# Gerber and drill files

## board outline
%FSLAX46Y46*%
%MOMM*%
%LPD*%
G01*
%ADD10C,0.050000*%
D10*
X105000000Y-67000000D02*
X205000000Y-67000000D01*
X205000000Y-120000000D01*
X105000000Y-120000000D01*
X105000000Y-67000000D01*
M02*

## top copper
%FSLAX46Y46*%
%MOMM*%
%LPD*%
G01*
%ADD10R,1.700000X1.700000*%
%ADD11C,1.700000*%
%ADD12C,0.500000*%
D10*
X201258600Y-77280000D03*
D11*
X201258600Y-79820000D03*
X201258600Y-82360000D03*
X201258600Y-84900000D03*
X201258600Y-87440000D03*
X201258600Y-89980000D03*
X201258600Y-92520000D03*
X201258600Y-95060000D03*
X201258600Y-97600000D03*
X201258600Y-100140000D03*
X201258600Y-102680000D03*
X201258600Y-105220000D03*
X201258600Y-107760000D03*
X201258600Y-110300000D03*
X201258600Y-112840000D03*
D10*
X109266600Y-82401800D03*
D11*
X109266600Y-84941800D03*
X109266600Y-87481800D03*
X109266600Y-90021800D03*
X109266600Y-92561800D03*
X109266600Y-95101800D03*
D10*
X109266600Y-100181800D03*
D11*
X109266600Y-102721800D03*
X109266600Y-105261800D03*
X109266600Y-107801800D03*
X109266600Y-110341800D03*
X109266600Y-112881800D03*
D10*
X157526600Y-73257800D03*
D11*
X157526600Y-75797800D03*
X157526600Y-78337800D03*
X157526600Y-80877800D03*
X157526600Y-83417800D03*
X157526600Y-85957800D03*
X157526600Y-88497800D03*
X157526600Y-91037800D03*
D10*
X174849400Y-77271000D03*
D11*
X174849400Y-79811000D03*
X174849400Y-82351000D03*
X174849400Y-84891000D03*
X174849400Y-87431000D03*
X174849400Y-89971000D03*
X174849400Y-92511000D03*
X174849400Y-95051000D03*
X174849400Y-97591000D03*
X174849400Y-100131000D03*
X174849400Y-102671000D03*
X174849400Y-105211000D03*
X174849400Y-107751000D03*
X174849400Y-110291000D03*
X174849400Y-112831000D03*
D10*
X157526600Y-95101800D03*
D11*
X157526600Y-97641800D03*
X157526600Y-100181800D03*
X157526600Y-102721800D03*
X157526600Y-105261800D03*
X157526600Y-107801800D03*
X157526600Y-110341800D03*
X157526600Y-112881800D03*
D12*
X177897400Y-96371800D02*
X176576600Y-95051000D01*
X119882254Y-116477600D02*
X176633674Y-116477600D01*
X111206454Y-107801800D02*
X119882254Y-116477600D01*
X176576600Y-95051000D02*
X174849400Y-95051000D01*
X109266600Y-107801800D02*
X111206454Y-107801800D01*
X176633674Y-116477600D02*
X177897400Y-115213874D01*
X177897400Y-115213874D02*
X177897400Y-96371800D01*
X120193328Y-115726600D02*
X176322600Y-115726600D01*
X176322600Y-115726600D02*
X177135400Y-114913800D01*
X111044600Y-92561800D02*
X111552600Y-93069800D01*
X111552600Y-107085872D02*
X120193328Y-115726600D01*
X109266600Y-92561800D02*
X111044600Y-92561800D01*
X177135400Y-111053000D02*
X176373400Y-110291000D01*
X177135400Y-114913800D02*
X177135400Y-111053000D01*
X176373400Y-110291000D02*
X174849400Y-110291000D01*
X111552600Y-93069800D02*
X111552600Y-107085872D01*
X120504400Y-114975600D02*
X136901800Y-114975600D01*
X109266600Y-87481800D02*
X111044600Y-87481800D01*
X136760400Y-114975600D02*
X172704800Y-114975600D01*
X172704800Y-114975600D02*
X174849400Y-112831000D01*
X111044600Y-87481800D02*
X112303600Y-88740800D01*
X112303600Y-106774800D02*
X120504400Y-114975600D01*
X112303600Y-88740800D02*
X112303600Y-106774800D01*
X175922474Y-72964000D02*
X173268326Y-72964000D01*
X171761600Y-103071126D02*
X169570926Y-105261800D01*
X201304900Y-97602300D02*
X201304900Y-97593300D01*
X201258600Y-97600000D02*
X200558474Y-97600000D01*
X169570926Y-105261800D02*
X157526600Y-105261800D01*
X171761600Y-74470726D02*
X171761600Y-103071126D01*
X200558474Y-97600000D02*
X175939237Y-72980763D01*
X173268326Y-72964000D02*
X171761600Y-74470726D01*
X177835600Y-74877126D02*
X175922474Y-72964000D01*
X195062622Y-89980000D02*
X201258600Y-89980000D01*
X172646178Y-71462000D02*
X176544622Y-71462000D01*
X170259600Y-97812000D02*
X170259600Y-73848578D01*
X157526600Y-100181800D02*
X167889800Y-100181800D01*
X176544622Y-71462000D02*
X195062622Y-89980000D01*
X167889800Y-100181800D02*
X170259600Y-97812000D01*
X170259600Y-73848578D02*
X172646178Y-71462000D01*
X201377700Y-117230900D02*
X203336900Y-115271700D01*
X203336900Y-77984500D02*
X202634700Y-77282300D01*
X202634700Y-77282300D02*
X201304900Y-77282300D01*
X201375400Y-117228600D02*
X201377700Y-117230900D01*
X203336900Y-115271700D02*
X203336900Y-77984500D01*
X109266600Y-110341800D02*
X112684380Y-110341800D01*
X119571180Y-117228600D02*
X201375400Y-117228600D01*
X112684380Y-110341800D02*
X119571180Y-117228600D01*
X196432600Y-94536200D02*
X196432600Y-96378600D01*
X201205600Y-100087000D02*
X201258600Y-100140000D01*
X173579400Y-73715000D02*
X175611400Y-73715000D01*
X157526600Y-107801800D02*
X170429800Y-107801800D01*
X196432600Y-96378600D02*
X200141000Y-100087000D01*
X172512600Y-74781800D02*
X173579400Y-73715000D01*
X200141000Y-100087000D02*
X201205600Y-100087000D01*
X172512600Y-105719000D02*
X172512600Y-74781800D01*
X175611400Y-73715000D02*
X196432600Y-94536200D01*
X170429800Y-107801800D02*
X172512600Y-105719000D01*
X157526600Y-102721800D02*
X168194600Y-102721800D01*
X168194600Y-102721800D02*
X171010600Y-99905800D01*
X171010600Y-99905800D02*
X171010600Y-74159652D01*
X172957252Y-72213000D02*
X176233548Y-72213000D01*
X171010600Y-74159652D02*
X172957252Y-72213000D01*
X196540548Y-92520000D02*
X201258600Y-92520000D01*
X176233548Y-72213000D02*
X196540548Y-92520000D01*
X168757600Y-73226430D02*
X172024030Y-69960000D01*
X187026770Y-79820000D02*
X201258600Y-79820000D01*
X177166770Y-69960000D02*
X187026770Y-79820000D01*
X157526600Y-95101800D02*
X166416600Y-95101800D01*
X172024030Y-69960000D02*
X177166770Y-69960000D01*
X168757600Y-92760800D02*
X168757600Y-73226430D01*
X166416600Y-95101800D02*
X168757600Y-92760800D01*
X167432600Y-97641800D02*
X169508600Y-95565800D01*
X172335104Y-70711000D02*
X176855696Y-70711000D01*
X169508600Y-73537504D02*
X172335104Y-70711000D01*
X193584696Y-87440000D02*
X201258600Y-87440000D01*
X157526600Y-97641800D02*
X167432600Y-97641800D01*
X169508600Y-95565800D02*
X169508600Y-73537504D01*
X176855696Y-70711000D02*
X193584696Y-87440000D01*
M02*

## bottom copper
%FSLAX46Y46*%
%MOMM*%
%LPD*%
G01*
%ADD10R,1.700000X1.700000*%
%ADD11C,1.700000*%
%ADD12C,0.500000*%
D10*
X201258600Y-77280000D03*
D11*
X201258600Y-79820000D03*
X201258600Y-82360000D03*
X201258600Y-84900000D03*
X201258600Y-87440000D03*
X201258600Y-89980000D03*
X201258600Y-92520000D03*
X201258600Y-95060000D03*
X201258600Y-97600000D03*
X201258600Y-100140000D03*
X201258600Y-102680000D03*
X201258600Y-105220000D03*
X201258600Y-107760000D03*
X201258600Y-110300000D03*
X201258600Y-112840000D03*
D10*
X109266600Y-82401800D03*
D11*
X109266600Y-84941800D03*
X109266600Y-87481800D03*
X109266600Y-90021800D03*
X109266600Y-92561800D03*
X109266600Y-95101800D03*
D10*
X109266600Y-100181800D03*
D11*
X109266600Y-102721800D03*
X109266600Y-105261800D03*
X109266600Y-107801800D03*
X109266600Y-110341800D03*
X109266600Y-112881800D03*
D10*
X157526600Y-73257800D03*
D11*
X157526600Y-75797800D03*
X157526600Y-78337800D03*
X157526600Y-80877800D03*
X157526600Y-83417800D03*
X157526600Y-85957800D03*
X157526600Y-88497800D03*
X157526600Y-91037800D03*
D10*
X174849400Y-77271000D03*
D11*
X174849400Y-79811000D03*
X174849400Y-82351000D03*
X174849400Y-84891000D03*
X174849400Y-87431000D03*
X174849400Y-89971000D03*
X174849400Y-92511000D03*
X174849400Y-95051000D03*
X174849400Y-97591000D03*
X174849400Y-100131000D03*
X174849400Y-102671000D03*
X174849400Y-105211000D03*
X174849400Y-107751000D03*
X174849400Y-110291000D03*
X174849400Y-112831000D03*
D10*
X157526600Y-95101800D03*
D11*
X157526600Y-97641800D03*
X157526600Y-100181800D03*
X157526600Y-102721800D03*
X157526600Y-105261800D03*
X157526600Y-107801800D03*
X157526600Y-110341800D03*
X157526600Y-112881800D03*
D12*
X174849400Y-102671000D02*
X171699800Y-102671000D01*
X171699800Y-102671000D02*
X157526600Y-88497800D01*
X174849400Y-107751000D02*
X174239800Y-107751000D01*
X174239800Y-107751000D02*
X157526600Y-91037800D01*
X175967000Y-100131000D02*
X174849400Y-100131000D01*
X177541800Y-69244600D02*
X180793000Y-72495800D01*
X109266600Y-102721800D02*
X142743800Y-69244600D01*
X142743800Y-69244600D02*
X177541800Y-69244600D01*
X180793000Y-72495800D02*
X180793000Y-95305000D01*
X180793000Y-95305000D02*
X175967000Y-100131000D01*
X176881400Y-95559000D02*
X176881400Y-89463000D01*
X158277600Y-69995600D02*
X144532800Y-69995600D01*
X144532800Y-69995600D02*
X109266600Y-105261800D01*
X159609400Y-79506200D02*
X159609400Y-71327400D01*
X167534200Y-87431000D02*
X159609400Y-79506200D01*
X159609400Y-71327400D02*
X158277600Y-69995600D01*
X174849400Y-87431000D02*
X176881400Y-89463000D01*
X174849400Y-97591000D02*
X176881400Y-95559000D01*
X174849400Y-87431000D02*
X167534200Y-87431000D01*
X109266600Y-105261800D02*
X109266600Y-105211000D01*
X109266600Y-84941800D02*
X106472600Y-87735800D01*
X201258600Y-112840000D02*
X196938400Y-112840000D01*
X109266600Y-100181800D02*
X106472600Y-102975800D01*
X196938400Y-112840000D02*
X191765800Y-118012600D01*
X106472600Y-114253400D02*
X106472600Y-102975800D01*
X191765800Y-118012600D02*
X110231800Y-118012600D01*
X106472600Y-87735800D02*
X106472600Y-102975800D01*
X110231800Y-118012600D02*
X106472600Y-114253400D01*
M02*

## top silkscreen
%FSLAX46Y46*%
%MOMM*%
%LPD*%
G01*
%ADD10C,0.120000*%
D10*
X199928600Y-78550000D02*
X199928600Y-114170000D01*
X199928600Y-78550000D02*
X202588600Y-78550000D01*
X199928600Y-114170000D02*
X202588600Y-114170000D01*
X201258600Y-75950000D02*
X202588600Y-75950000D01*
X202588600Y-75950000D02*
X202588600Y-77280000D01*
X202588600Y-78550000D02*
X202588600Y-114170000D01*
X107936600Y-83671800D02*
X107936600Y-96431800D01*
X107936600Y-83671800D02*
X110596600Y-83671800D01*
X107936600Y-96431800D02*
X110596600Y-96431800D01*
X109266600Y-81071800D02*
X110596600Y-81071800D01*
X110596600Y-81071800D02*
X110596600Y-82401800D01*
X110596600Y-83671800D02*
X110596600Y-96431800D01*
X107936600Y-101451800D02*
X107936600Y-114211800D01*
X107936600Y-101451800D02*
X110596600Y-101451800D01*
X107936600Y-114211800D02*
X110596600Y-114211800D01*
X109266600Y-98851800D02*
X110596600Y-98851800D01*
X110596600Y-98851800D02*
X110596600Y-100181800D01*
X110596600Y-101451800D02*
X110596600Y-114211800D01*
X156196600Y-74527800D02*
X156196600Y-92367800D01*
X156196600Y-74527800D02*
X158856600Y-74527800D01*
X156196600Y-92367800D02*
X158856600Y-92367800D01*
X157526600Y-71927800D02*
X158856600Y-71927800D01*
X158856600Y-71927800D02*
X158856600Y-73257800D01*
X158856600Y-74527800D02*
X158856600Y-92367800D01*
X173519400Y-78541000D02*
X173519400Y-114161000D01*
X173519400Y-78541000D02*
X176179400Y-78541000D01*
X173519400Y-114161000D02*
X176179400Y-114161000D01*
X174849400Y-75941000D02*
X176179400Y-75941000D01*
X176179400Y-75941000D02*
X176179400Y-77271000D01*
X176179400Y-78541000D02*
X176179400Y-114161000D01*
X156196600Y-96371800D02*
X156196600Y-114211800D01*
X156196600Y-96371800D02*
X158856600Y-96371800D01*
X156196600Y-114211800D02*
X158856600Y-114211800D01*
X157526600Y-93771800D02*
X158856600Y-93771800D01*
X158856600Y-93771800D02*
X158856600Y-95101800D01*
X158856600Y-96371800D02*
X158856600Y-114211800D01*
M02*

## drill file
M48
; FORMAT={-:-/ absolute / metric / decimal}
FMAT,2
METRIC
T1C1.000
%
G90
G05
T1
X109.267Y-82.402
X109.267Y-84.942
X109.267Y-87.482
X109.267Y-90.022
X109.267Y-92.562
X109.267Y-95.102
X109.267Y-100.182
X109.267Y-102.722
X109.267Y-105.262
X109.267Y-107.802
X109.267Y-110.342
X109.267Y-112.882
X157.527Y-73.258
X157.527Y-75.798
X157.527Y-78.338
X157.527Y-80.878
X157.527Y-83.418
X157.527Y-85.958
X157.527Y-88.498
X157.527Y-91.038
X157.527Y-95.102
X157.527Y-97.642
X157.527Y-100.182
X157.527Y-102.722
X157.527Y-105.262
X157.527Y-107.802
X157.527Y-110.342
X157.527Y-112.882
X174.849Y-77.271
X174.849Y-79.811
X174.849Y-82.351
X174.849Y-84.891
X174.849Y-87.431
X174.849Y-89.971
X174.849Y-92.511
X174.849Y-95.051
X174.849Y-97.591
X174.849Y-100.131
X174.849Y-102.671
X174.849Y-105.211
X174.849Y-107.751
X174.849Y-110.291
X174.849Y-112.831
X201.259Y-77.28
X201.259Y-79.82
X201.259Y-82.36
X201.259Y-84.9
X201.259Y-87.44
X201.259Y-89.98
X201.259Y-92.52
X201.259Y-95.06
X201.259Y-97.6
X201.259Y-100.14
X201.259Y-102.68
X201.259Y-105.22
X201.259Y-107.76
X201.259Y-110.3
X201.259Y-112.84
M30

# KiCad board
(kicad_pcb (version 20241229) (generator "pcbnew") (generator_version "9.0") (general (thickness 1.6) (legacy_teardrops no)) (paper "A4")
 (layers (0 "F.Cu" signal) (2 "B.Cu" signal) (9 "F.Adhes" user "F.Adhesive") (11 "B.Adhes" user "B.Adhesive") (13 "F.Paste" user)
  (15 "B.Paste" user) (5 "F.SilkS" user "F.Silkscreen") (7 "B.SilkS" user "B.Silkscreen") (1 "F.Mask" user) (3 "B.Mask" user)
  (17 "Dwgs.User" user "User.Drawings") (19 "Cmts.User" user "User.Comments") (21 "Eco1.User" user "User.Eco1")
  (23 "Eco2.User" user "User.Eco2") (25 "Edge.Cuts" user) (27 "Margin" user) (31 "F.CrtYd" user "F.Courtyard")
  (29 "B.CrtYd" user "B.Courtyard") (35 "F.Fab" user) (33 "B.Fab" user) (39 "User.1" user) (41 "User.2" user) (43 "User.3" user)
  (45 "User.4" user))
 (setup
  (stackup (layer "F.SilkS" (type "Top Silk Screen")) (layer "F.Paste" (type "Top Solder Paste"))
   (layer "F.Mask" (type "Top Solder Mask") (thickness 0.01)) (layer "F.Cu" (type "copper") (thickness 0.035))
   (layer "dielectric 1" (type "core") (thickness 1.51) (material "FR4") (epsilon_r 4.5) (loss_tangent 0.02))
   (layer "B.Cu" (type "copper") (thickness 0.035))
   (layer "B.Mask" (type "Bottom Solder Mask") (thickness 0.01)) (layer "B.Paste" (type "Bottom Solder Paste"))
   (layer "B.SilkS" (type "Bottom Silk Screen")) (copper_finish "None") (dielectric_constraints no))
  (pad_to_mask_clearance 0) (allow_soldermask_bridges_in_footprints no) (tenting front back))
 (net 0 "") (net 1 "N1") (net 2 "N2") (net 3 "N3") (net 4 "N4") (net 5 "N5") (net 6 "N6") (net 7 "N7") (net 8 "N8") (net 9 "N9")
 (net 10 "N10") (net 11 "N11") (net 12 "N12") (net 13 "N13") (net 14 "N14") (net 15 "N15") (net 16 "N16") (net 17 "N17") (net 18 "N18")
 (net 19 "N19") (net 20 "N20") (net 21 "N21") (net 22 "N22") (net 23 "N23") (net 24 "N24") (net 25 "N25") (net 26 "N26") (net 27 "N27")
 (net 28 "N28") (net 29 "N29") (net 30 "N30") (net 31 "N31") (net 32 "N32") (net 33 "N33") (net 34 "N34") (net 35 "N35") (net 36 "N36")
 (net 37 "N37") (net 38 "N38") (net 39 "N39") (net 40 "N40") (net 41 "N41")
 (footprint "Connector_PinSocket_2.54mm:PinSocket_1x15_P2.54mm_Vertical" (layer "F.Cu") (at 201.2586 77.28)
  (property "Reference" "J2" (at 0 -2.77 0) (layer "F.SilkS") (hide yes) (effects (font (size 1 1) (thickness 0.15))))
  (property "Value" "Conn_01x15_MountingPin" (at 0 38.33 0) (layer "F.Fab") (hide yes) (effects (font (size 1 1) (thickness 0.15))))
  (fp_line (start -1.33 1.27) (end -1.33 36.89) (stroke (width 0.12) (type solid)) (layer "F.SilkS"))
  (fp_line (start -1.33 1.27) (end 1.33 1.27) (stroke (width 0.12) (type solid)) (layer "F.SilkS"))
  (fp_line (start -1.33 36.89) (end 1.33 36.89) (stroke (width 0.12) (type solid)) (layer "F.SilkS"))
  (fp_line (start 0 -1.33) (end 1.33 -1.33) (stroke (width 0.12) (type solid)) (layer "F.SilkS"))
  (fp_line (start 1.33 -1.33) (end 1.33 0) (stroke (width 0.12) (type solid)) (layer "F.SilkS"))
  (fp_line (start 1.33 1.27) (end 1.33 36.89) (stroke (width 0.12) (type solid)) (layer "F.SilkS"))
  (pad "1" thru_hole rect (at 0 0) (size 1.7 1.7) (drill 1) (layers "*.Cu" "*.Mask") (remove_unused_layers no) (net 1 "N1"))
  (pad "2" thru_hole circle (at 0 2.54) (size 1.7 1.7) (drill 1) (layers "*.Cu" "*.Mask") (remove_unused_layers no) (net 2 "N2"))
  (pad "3" thru_hole circle (at 0 5.08) (size 1.7 1.7) (drill 1) (layers "*.Cu" "*.Mask") (remove_unused_layers no) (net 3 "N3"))
  (pad "4" thru_hole circle (at 0 7.62) (size 1.7 1.7) (drill 1) (layers "*.Cu" "*.Mask") (remove_unused_layers no) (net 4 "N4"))
  (pad "5" thru_hole circle (at 0 10.16) (size 1.7 1.7) (drill 1) (layers "*.Cu" "*.Mask") (remove_unused_layers no) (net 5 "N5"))
  (pad "6" thru_hole circle (at 0 12.7) (size 1.7 1.7) (drill 1) (layers "*.Cu" "*.Mask") (remove_unused_layers no) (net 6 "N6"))
  (pad "7" thru_hole circle (at 0 15.24) (size 1.7 1.7) (drill 1) (layers "*.Cu" "*.Mask") (remove_unused_layers no) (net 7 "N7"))
  (pad "8" thru_hole circle (at 0 17.78) (size 1.7 1.7) (drill 1) (layers "*.Cu" "*.Mask") (remove_unused_layers no) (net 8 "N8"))
  (pad "9" thru_hole circle (at 0 20.32) (size 1.7 1.7) (drill 1) (layers "*.Cu" "*.Mask") (remove_unused_layers no) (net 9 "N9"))
  (pad "10" thru_hole circle (at 0 22.86) (size 1.7 1.7) (drill 1) (layers "*.Cu" "*.Mask") (remove_unused_layers no) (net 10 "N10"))
  (pad "11" thru_hole circle (at 0 25.4) (size 1.7 1.7) (drill 1) (layers "*.Cu" "*.Mask") (remove_unused_layers no) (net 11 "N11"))
  (pad "12" thru_hole circle (at 0 27.94) (size 1.7 1.7) (drill 1) (layers "*.Cu" "*.Mask") (remove_unused_layers no) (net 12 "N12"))
  (pad "13" thru_hole circle (at 0 30.48) (size 1.7 1.7) (drill 1) (layers "*.Cu" "*.Mask") (remove_unused_layers no) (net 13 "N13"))
  (pad "14" thru_hole circle (at 0 33.02) (size 1.7 1.7) (drill 1) (layers "*.Cu" "*.Mask") (remove_unused_layers no) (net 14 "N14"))
  (pad "15" thru_hole circle (at 0 35.56) (size 1.7 1.7) (drill 1) (layers "*.Cu" "*.Mask") (remove_unused_layers no) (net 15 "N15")))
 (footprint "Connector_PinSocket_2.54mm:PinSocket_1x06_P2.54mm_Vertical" (layer "F.Cu") (at 109.2666 82.4018)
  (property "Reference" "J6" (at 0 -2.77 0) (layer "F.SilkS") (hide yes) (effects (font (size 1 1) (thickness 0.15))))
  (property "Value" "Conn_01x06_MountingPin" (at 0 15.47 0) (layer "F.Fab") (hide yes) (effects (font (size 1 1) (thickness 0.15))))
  (fp_line (start -1.33 1.27) (end -1.33 14.03) (stroke (width 0.12) (type solid)) (layer "F.SilkS"))
  (fp_line (start -1.33 1.27) (end 1.33 1.27) (stroke (width 0.12) (type solid)) (layer "F.SilkS"))
  (fp_line (start -1.33 14.03) (end 1.33 14.03) (stroke (width 0.12) (type solid)) (layer "F.SilkS"))
  (fp_line (start 0 -1.33) (end 1.33 -1.33) (stroke (width 0.12) (type solid)) (layer "F.SilkS"))
  (fp_line (start 1.33 -1.33) (end 1.33 0) (stroke (width 0.12) (type solid)) (layer "F.SilkS"))
  (fp_line (start 1.33 1.27) (end 1.33 14.03) (stroke (width 0.12) (type solid)) (layer "F.SilkS"))
  (pad "1" thru_hole rect (at 0 0) (size 1.7 1.7) (drill 1) (layers "*.Cu" "*.Mask") (remove_unused_layers no) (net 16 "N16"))
  (pad "2" thru_hole circle (at 0 2.54) (size 1.7 1.7) (drill 1) (layers "*.Cu" "*.Mask") (remove_unused_layers no) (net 15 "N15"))
  (pad "3" thru_hole circle (at 0 5.08) (size 1.7 1.7) (drill 1) (layers "*.Cu" "*.Mask") (remove_unused_layers no) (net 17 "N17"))
  (pad "4" thru_hole circle (at 0 7.62) (size 1.7 1.7) (drill 1) (layers "*.Cu" "*.Mask") (remove_unused_layers no) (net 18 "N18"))
  (pad "5" thru_hole circle (at 0 10.16) (size 1.7 1.7) (drill 1) (layers "*.Cu" "*.Mask") (remove_unused_layers no) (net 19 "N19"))
  (pad "6" thru_hole circle (at 0 12.7) (size 1.7 1.7) (drill 1) (layers "*.Cu" "*.Mask") (remove_unused_layers no) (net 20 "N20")))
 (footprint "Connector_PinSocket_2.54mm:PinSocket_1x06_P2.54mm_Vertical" (layer "F.Cu") (at 109.2666 100.1818)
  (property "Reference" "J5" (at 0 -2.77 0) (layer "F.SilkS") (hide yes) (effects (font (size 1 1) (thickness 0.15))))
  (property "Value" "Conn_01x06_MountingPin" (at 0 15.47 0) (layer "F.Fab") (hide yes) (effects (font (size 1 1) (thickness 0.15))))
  (fp_line (start -1.33 1.27) (end -1.33 14.03) (stroke (width 0.12) (type solid)) (layer "F.SilkS"))
  (fp_line (start -1.33 1.27) (end 1.33 1.27) (stroke (width 0.12) (type solid)) (layer "F.SilkS"))
  (fp_line (start -1.33 14.03) (end 1.33 14.03) (stroke (width 0.12) (type solid)) (layer "F.SilkS"))
  (fp_line (start 0 -1.33) (end 1.33 -1.33) (stroke (width 0.12) (type solid)) (layer "F.SilkS"))
  (fp_line (start 1.33 -1.33) (end 1.33 0) (stroke (width 0.12) (type solid)) (layer "F.SilkS"))
  (fp_line (start 1.33 1.27) (end 1.33 14.03) (stroke (width 0.12) (type solid)) (layer "F.SilkS"))
  (pad "1" thru_hole rect (at 0 0) (size 1.7 1.7) (drill 1) (layers "*.Cu" "*.Mask") (remove_unused_layers no) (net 15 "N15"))
  (pad "2" thru_hole circle (at 0 2.54) (size 1.7 1.7) (drill 1) (layers "*.Cu" "*.Mask") (remove_unused_layers no) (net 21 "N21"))
  (pad "3" thru_hole circle (at 0 5.08) (size 1.7 1.7) (drill 1) (layers "*.Cu" "*.Mask") (remove_unused_layers no) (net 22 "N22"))
  (pad "4" thru_hole circle (at 0 7.62) (size 1.7 1.7) (drill 1) (layers "*.Cu" "*.Mask") (remove_unused_layers no) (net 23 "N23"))
  (pad "5" thru_hole circle (at 0 10.16) (size 1.7 1.7) (drill 1) (layers "*.Cu" "*.Mask") (remove_unused_layers no) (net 1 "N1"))
  (pad "6" thru_hole circle (at 0 12.7) (size 1.7 1.7) (drill 1) (layers "*.Cu" "*.Mask") (remove_unused_layers no) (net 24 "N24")))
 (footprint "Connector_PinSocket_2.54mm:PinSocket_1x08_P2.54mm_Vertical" (layer "F.Cu") (at 157.5266 73.2578)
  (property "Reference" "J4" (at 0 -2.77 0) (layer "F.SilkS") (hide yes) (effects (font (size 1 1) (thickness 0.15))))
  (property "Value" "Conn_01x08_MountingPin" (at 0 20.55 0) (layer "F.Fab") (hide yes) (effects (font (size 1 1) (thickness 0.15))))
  (fp_line (start -1.33 1.27) (end -1.33 19.11) (stroke (width 0.12) (type solid)) (layer "F.SilkS"))
  (fp_line (start -1.33 1.27) (end 1.33 1.27) (stroke (width 0.12) (type solid)) (layer "F.SilkS"))
  (fp_line (start -1.33 19.11) (end 1.33 19.11) (stroke (width 0.12) (type solid)) (layer "F.SilkS"))
  (fp_line (start 0 -1.33) (end 1.33 -1.33) (stroke (width 0.12) (type solid)) (layer "F.SilkS"))
  (fp_line (start 1.33 -1.33) (end 1.33 0) (stroke (width 0.12) (type solid)) (layer "F.SilkS"))
  (fp_line (start 1.33 1.27) (end 1.33 19.11) (stroke (width 0.12) (type solid)) (layer "F.SilkS"))
  (pad "1" thru_hole rect (at 0 0) (size 1.7 1.7) (drill 1) (layers "*.Cu" "*.Mask") (remove_unused_layers no) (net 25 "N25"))
  (pad "2" thru_hole circle (at 0 2.54) (size 1.7 1.7) (drill 1) (layers "*.Cu" "*.Mask") (remove_unused_layers no) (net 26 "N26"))
  (pad "3" thru_hole circle (at 0 5.08) (size 1.7 1.7) (drill 1) (layers "*.Cu" "*.Mask") (remove_unused_layers no) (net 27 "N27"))
  (pad "4" thru_hole circle (at 0 7.62) (size 1.7 1.7) (drill 1) (layers "*.Cu" "*.Mask") (remove_unused_layers no) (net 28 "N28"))
  (pad "5" thru_hole circle (at 0 10.16) (size 1.7 1.7) (drill 1) (layers "*.Cu" "*.Mask") (remove_unused_layers no) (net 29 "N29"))
  (pad "6" thru_hole circle (at 0 12.7) (size 1.7 1.7) (drill 1) (layers "*.Cu" "*.Mask") (remove_unused_layers no) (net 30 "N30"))
  (pad "7" thru_hole circle (at 0 15.24) (size 1.7 1.7) (drill 1) (layers "*.Cu" "*.Mask") (remove_unused_layers no) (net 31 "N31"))
  (pad "8" thru_hole circle (at 0 17.78) (size 1.7 1.7) (drill 1) (layers "*.Cu" "*.Mask") (remove_unused_layers no) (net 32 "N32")))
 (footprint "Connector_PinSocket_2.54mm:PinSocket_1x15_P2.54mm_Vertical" (layer "F.Cu") (at 174.8494 77.271)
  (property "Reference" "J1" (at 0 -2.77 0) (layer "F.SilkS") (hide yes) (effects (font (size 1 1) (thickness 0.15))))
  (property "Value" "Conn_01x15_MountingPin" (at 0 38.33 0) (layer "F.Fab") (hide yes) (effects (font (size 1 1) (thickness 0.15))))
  (fp_line (start -1.33 1.27) (end -1.33 36.89) (stroke (width 0.12) (type solid)) (layer "F.SilkS"))
  (fp_line (start -1.33 1.27) (end 1.33 1.27) (stroke (width 0.12) (type solid)) (layer "F.SilkS"))
  (fp_line (start -1.33 36.89) (end 1.33 36.89) (stroke (width 0.12) (type solid)) (layer "F.SilkS"))
  (fp_line (start 0 -1.33) (end 1.33 -1.33) (stroke (width 0.12) (type solid)) (layer "F.SilkS"))
  (fp_line (start 1.33 -1.33) (end 1.33 0) (stroke (width 0.12) (type solid)) (layer "F.SilkS"))
  (fp_line (start 1.33 1.27) (end 1.33 36.89) (stroke (width 0.12) (type solid)) (layer "F.SilkS"))
  (pad "1" thru_hole rect (at 0 0) (size 1.7 1.7) (drill 1) (layers "*.Cu" "*.Mask") (remove_unused_layers no) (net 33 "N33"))
  (pad "2" thru_hole circle (at 0 2.54) (size 1.7 1.7) (drill 1) (layers "*.Cu" "*.Mask") (remove_unused_layers no) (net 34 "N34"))
  (pad "3" thru_hole circle (at 0 5.08) (size 1.7 1.7) (drill 1) (layers "*.Cu" "*.Mask") (remove_unused_layers no) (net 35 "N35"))
  (pad "4" thru_hole circle (at 0 7.62) (size 1.7 1.7) (drill 1) (layers "*.Cu" "*.Mask") (remove_unused_layers no) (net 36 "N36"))
  (pad "5" thru_hole circle (at 0 10.16) (size 1.7 1.7) (drill 1) (layers "*.Cu" "*.Mask") (remove_unused_layers no) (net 22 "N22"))
  (pad "6" thru_hole circle (at 0 12.7) (size 1.7 1.7) (drill 1) (layers "*.Cu" "*.Mask") (remove_unused_layers no) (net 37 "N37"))
  (pad "7" thru_hole circle (at 0 15.24) (size 1.7 1.7) (drill 1) (layers "*.Cu" "*.Mask") (remove_unused_layers no) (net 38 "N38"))
  (pad "8" thru_hole circle (at 0 17.78) (size 1.7 1.7) (drill 1) (layers "*.Cu" "*.Mask") (remove_unused_layers no) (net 23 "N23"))
  (pad "9" thru_hole circle (at 0 20.32) (size 1.7 1.7) (drill 1) (layers "*.Cu" "*.Mask") (remove_unused_layers no) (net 22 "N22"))
  (pad "10" thru_hole circle (at 0 22.86) (size 1.7 1.7) (drill 1) (layers "*.Cu" "*.Mask") (remove_unused_layers no) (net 21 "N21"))
  (pad "11" thru_hole circle (at 0 25.4) (size 1.7 1.7) (drill 1) (layers "*.Cu" "*.Mask") (remove_unused_layers no) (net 31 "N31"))
  (pad "12" thru_hole circle (at 0 27.94) (size 1.7 1.7) (drill 1) (layers "*.Cu" "*.Mask") (remove_unused_layers no) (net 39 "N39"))
  (pad "13" thru_hole circle (at 0 30.48) (size 1.7 1.7) (drill 1) (layers "*.Cu" "*.Mask") (remove_unused_layers no) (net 32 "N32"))
  (pad "14" thru_hole circle (at 0 33.02) (size 1.7 1.7) (drill 1) (layers "*.Cu" "*.Mask") (remove_unused_layers no) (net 19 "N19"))
  (pad "15" thru_hole circle (at 0 35.56) (size 1.7 1.7) (drill 1) (layers "*.Cu" "*.Mask") (remove_unused_layers no) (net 17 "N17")))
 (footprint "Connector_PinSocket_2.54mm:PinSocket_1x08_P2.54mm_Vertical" (layer "F.Cu") (at 157.5266 95.1018)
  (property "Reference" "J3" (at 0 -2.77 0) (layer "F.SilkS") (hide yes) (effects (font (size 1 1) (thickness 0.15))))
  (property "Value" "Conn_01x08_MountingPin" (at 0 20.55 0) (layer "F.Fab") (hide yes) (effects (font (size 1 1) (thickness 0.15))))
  (fp_line (start -1.33 1.27) (end -1.33 19.11) (stroke (width 0.12) (type solid)) (layer "F.SilkS"))
  (fp_line (start -1.33 1.27) (end 1.33 1.27) (stroke (width 0.12) (type solid)) (layer "F.SilkS"))
  (fp_line (start -1.33 19.11) (end 1.33 19.11) (stroke (width 0.12) (type solid)) (layer "F.SilkS"))
  (fp_line (start 0 -1.33) (end 1.33 -1.33) (stroke (width 0.12) (type solid)) (layer "F.SilkS"))
  (fp_line (start 1.33 -1.33) (end 1.33 0) (stroke (width 0.12) (type solid)) (layer "F.SilkS"))
  (fp_line (start 1.33 1.27) (end 1.33 19.11) (stroke (width 0.12) (type solid)) (layer "F.SilkS"))
  (pad "1" thru_hole rect (at 0 0) (size 1.7 1.7) (drill 1) (layers "*.Cu" "*.Mask") (remove_unused_layers no) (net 2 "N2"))
  (pad "2" thru_hole circle (at 0 2.54) (size 1.7 1.7) (drill 1) (layers "*.Cu" "*.Mask") (remove_unused_layers no) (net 5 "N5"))
  (pad "3" thru_hole circle (at 0 5.08) (size 1.7 1.7) (drill 1) (layers "*.Cu" "*.Mask") (remove_unused_layers no) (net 6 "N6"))
  (pad "4" thru_hole circle (at 0 7.62) (size 1.7 1.7) (drill 1) (layers "*.Cu" "*.Mask") (remove_unused_layers no) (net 7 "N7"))
  (pad "5" thru_hole circle (at 0 10.16) (size 1.7 1.7) (drill 1) (layers "*.Cu" "*.Mask") (remove_unused_layers no) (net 9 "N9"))
  (pad "6" thru_hole circle (at 0 12.7) (size 1.7 1.7) (drill 1) (layers "*.Cu" "*.Mask") (remove_unused_layers no) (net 10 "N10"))
  (pad "7" thru_hole circle (at 0 15.24) (size 1.7 1.7) (drill 1) (layers "*.Cu" "*.Mask") (remove_unused_layers no) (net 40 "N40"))
  (pad "8" thru_hole circle (at 0 17.78) (size 1.7 1.7) (drill 1) (layers "*.Cu" "*.Mask") (remove_unused_layers no) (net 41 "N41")))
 (gr_rect (start 105 67) (end 205 120) (stroke (width 0.05) (type solid)) (fill no) (layer "Edge.Cuts"))
 (segment (start 174.8494 102.671) (end 171.6998 102.671) (width 0.5) (layer "B.Cu") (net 31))
 (segment (start 171.6998 102.671) (end 157.5266 88.4978) (width 0.5) (layer "B.Cu") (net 31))
 (segment (start 174.8494 107.751) (end 174.2398 107.751) (width 0.5) (layer "B.Cu") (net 32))
 (segment (start 174.2398 107.751) (end 157.5266 91.0378) (width 0.5) (layer "B.Cu") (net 32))
 (segment (start 177.8974 96.3718) (end 176.5766 95.051) (width 0.5) (layer "F.Cu") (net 23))
 (segment (start 119.882254 116.4776) (end 176.633674 116.4776) (width 0.5) (layer "F.Cu") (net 23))
 (segment (start 111.206454 107.8018) (end 119.882254 116.4776) (width 0.5) (layer "F.Cu") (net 23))
 (segment (start 176.5766 95.051) (end 174.8494 95.051) (width 0.5) (layer "F.Cu") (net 23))
 (segment (start 109.2666 107.8018) (end 111.206454 107.8018) (width 0.5) (layer "F.Cu") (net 23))
 (segment (start 176.633674 116.4776) (end 177.8974 115.213874) (width 0.5) (layer "F.Cu") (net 23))
 (segment (start 177.8974 115.213874) (end 177.8974 96.3718) (width 0.5) (layer "F.Cu") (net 23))
 (segment (start 120.193328 115.7266) (end 176.3226 115.7266) (width 0.5) (layer "F.Cu") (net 19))
 (segment (start 176.3226 115.7266) (end 177.1354 114.9138) (width 0.5) (layer "F.Cu") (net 19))
 (segment (start 111.0446 92.5618) (end 111.5526 93.0698) (width 0.5) (layer "F.Cu") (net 19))
 (segment (start 111.5526 107.085872) (end 120.193328 115.7266) (width 0.5) (layer "F.Cu") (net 19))
 (segment (start 109.2666 92.5618) (end 111.0446 92.5618) (width 0.5) (layer "F.Cu") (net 19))
 (segment (start 177.1354 111.053) (end 176.3734 110.291) (width 0.5) (layer "F.Cu") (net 19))
 (segment (start 177.1354 114.9138) (end 177.1354 111.053) (width 0.5) (layer "F.Cu") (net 19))
 (segment (start 176.3734 110.291) (end 174.8494 110.291) (width 0.5) (layer "F.Cu") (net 19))
 (segment (start 111.5526 93.0698) (end 111.5526 107.085872) (width 0.5) (layer "F.Cu") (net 19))
 (segment (start 175.967 100.131) (end 174.8494 100.131) (width 0.5) (layer "B.Cu") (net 21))
 (segment (start 177.5418 69.2446) (end 180.793 72.4958) (width 0.5) (layer "B.Cu") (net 21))
 (segment (start 109.2666 102.7218) (end 142.7438 69.2446) (width 0.5) (layer "B.Cu") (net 21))
 (segment (start 142.7438 69.2446) (end 177.5418 69.2446) (width 0.5) (layer "B.Cu") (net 21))
 (segment (start 180.793 72.4958) (end 180.793 95.305) (width 0.5) (layer "B.Cu") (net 21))
 (segment (start 180.793 95.305) (end 175.967 100.131) (width 0.5) (layer "B.Cu") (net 21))
 (segment (start 176.8814 95.559) (end 176.8814 89.463) (width 0.5) (layer "B.Cu") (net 22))
 (segment (start 158.2776 69.9956) (end 144.5328 69.9956) (width 0.5) (layer "B.Cu") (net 22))
 (segment (start 144.5328 69.9956) (end 109.2666 105.2618) (width 0.5) (layer "B.Cu") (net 22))
 (segment (start 159.6094 79.5062) (end 159.6094 71.3274) (width 0.5) (layer "B.Cu") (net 22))
 (segment (start 167.5342 87.431) (end 159.6094 79.5062) (width 0.5) (layer "B.Cu") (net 22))
 (segment (start 159.6094 71.3274) (end 158.2776 69.9956) (width 0.5) (layer "B.Cu") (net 22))
 (segment (start 174.8494 87.431) (end 176.8814 89.463) (width 0.5) (layer "B.Cu") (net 22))
 (segment (start 174.8494 97.591) (end 176.8814 95.559) (width 0.5) (layer "B.Cu") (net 22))
 (segment (start 174.8494 87.431) (end 167.5342 87.431) (width 0.5) (layer "B.Cu") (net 22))
 (segment (start 109.2666 105.2618) (end 109.2666 105.211) (width 0.5) (layer "B.Cu") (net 22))
 (segment (start 120.5044 114.9756) (end 136.9018 114.9756) (width 0.5) (layer "F.Cu") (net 17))
 (segment (start 109.2666 87.4818) (end 111.0446 87.4818) (width 0.5) (layer "F.Cu") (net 17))
 (segment (start 136.7604 114.9756) (end 172.7048 114.9756) (width 0.5) (layer "F.Cu") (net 17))
 (segment (start 172.7048 114.9756) (end 174.8494 112.831) (width 0.5) (layer "F.Cu") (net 17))
 (segment (start 111.0446 87.4818) (end 112.3036 88.7408) (width 0.5) (layer "F.Cu") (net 17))
 (segment (start 112.3036 106.7748) (end 120.5044 114.9756) (width 0.5) (layer "F.Cu") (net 17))
 (segment (start 112.3036 88.7408) (end 112.3036 106.7748) (width 0.5) (layer "F.Cu") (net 17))
 (segment (start 109.2666 84.9418) (end 106.4726 87.7358) (width 0.5) (layer "B.Cu") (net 15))
 (segment (start 201.2586 112.84) (end 196.9384 112.84) (width 0.5) (layer "B.Cu") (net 15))
 (segment (start 109.2666 100.1818) (end 106.4726 102.9758) (width 0.5) (layer "B.Cu") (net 15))
 (segment (start 196.9384 112.84) (end 191.7658 118.0126) (width 0.5) (layer "B.Cu") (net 15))
 (segment (start 106.4726 114.2534) (end 106.4726 102.9758) (width 0.5) (layer "B.Cu") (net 15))
 (segment (start 191.7658 118.0126) (end 110.2318 118.0126) (width 0.5) (layer "B.Cu") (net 15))
 (segment (start 106.4726 87.7358) (end 106.4726 102.9758) (width 0.5) (layer "B.Cu") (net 15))
 (segment (start 110.2318 118.0126) (end 106.4726 114.2534) (width 0.5) (layer "B.Cu") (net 15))
 (segment (start 175.922474 72.964) (end 173.268326 72.964) (width 0.5) (layer "F.Cu") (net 9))
 (segment (start 171.7616 103.071126) (end 169.570926 105.2618) (width 0.5) (layer "F.Cu") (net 9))
 (segment (start 201.3049 97.6023) (end 201.3049 97.5933) (width 0.5) (layer "F.Cu") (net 9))
 (segment (start 201.2586 97.6) (end 200.558474 97.6) (width 0.5) (layer "F.Cu") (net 9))
 (segment (start 169.570926 105.2618) (end 157.5266 105.2618) (width 0.5) (layer "F.Cu") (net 9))
 (segment (start 171.7616 74.470726) (end 171.7616 103.071126) (width 0.5) (layer "F.Cu") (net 9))
 (segment (start 200.558474 97.6) (end 175.939237 72.980763) (width 0.5) (layer "F.Cu") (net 9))
 (segment (start 173.268326 72.964) (end 171.7616 74.470726) (width 0.5) (layer "F.Cu") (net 9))
 (segment (start 177.8356 74.877126) (end 175.922474 72.964) (width 0.5) (layer "F.Cu") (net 9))
 (segment (start 195.062622 89.98) (end 201.2586 89.98) (width 0.5) (layer "F.Cu") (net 6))
 (segment (start 172.646178 71.462) (end 176.544622 71.462) (width 0.5) (layer "F.Cu") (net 6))
 (segment (start 170.2596 97.812) (end 170.2596 73.848578) (width 0.5) (layer "F.Cu") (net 6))
 (segment (start 157.5266 100.1818) (end 167.8898 100.1818) (width 0.5) (layer "F.Cu") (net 6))
 (segment (start 176.544622 71.462) (end 195.062622 89.98) (width 0.5) (layer "F.Cu") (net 6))
 (segment (start 167.8898 100.1818) (end 170.2596 97.812) (width 0.5) (layer "F.Cu") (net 6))
 (segment (start 170.2596 73.848578) (end 172.646178 71.462) (width 0.5) (layer "F.Cu") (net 6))
 (segment (start 201.3777 117.2309) (end 203.3369 115.2717) (width 0.5) (layer "F.Cu") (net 1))
 (segment (start 203.3369 77.9845) (end 202.6347 77.2823) (width 0.5) (layer "F.Cu") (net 1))
 (segment (start 202.6347 77.2823) (end 201.3049 77.2823) (width 0.5) (layer "F.Cu") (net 1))
 (segment (start 201.3754 117.2286) (end 201.3777 117.2309) (width 0.5) (layer "F.Cu") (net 1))
 (segment (start 203.3369 115.2717) (end 203.3369 77.9845) (width 0.5) (layer "F.Cu") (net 1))
 (segment (start 109.2666 110.3418) (end 112.68438 110.3418) (width 0.5) (layer "F.Cu") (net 1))
 (segment (start 119.57118 117.2286) (end 201.3754 117.2286) (width 0.5) (layer "F.Cu") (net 1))
 (segment (start 112.68438 110.3418) (end 119.57118 117.2286) (width 0.5) (layer "F.Cu") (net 1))
 (segment (start 196.4326 94.5362) (end 196.4326 96.3786) (width 0.5) (layer "F.Cu") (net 10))
 (segment (start 201.2056 100.087) (end 201.2586 100.14) (width 0.5) (layer "F.Cu") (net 10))
 (segment (start 173.5794 73.715) (end 175.6114 73.715) (width 0.5) (layer "F.Cu") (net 10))
 (segment (start 157.5266 107.8018) (end 170.4298 107.8018) (width 0.5) (layer "F.Cu") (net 10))
 (segment (start 196.4326 96.3786) (end 200.141 100.087) (width 0.5) (layer "F.Cu") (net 10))
 (segment (start 172.5126 74.7818) (end 173.5794 73.715) (width 0.5) (layer "F.Cu") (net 10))
 (segment (start 200.141 100.087) (end 201.2056 100.087) (width 0.5) (layer "F.Cu") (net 10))
 (segment (start 172.5126 105.719) (end 172.5126 74.7818) (width 0.5) (layer "F.Cu") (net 10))
 (segment (start 175.6114 73.715) (end 196.4326 94.5362) (width 0.5) (layer "F.Cu") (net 10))
 (segment (start 170.4298 107.8018) (end 172.5126 105.719) (width 0.5) (layer "F.Cu") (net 10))
 (segment (start 157.5266 102.7218) (end 168.1946 102.7218) (width 0.5) (layer "F.Cu") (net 7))
 (segment (start 168.1946 102.7218) (end 171.0106 99.9058) (width 0.5) (layer "F.Cu") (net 7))
 (segment (start 171.0106 99.9058) (end 171.0106 74.159652) (width 0.5) (layer "F.Cu") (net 7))
 (segment (start 172.957252 72.213) (end 176.233548 72.213) (width 0.5) (layer "F.Cu") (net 7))
 (segment (start 171.0106 74.159652) (end 172.957252 72.213) (width 0.5) (layer "F.Cu") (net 7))
 (segment (start 196.540548 92.52) (end 201.2586 92.52) (width 0.5) (layer "F.Cu") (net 7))
 (segment (start 176.233548 72.213) (end 196.540548 92.52) (width 0.5) (layer "F.Cu") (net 7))
 (segment (start 168.7576 73.22643) (end 172.02403 69.96) (width 0.5) (layer "F.Cu") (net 2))
 (segment (start 187.02677 79.82) (end 201.2586 79.82) (width 0.5) (layer "F.Cu") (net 2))
 (segment (start 177.16677 69.96) (end 187.02677 79.82) (width 0.5) (layer "F.Cu") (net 2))
 (segment (start 157.5266 95.1018) (end 166.4166 95.1018) (width 0.5) (layer "F.Cu") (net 2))
 (segment (start 172.02403 69.96) (end 177.16677 69.96) (width 0.5) (layer "F.Cu") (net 2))
 (segment (start 168.7576 92.7608) (end 168.7576 73.22643) (width 0.5) (layer "F.Cu") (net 2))
 (segment (start 166.4166 95.1018) (end 168.7576 92.7608) (width 0.5) (layer "F.Cu") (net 2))
 (segment (start 167.4326 97.6418) (end 169.5086 95.5658) (width 0.5) (layer "F.Cu") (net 5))
 (segment (start 172.335104 70.711) (end 176.855696 70.711) (width 0.5) (layer "F.Cu") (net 5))
 (segment (start 169.5086 73.537504) (end 172.335104 70.711) (width 0.5) (layer "F.Cu") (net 5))
 (segment (start 193.584696 87.44) (end 201.2586 87.44) (width 0.5) (layer "F.Cu") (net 5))
 (segment (start 157.5266 97.6418) (end 167.4326 97.6418) (width 0.5) (layer "F.Cu") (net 5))
 (segment (start 169.5086 95.5658) (end 169.5086 73.537504) (width 0.5) (layer "F.Cu") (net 5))
 (segment (start 176.855696 70.711) (end 193.584696 87.44) (width 0.5) (layer "F.Cu") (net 5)))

